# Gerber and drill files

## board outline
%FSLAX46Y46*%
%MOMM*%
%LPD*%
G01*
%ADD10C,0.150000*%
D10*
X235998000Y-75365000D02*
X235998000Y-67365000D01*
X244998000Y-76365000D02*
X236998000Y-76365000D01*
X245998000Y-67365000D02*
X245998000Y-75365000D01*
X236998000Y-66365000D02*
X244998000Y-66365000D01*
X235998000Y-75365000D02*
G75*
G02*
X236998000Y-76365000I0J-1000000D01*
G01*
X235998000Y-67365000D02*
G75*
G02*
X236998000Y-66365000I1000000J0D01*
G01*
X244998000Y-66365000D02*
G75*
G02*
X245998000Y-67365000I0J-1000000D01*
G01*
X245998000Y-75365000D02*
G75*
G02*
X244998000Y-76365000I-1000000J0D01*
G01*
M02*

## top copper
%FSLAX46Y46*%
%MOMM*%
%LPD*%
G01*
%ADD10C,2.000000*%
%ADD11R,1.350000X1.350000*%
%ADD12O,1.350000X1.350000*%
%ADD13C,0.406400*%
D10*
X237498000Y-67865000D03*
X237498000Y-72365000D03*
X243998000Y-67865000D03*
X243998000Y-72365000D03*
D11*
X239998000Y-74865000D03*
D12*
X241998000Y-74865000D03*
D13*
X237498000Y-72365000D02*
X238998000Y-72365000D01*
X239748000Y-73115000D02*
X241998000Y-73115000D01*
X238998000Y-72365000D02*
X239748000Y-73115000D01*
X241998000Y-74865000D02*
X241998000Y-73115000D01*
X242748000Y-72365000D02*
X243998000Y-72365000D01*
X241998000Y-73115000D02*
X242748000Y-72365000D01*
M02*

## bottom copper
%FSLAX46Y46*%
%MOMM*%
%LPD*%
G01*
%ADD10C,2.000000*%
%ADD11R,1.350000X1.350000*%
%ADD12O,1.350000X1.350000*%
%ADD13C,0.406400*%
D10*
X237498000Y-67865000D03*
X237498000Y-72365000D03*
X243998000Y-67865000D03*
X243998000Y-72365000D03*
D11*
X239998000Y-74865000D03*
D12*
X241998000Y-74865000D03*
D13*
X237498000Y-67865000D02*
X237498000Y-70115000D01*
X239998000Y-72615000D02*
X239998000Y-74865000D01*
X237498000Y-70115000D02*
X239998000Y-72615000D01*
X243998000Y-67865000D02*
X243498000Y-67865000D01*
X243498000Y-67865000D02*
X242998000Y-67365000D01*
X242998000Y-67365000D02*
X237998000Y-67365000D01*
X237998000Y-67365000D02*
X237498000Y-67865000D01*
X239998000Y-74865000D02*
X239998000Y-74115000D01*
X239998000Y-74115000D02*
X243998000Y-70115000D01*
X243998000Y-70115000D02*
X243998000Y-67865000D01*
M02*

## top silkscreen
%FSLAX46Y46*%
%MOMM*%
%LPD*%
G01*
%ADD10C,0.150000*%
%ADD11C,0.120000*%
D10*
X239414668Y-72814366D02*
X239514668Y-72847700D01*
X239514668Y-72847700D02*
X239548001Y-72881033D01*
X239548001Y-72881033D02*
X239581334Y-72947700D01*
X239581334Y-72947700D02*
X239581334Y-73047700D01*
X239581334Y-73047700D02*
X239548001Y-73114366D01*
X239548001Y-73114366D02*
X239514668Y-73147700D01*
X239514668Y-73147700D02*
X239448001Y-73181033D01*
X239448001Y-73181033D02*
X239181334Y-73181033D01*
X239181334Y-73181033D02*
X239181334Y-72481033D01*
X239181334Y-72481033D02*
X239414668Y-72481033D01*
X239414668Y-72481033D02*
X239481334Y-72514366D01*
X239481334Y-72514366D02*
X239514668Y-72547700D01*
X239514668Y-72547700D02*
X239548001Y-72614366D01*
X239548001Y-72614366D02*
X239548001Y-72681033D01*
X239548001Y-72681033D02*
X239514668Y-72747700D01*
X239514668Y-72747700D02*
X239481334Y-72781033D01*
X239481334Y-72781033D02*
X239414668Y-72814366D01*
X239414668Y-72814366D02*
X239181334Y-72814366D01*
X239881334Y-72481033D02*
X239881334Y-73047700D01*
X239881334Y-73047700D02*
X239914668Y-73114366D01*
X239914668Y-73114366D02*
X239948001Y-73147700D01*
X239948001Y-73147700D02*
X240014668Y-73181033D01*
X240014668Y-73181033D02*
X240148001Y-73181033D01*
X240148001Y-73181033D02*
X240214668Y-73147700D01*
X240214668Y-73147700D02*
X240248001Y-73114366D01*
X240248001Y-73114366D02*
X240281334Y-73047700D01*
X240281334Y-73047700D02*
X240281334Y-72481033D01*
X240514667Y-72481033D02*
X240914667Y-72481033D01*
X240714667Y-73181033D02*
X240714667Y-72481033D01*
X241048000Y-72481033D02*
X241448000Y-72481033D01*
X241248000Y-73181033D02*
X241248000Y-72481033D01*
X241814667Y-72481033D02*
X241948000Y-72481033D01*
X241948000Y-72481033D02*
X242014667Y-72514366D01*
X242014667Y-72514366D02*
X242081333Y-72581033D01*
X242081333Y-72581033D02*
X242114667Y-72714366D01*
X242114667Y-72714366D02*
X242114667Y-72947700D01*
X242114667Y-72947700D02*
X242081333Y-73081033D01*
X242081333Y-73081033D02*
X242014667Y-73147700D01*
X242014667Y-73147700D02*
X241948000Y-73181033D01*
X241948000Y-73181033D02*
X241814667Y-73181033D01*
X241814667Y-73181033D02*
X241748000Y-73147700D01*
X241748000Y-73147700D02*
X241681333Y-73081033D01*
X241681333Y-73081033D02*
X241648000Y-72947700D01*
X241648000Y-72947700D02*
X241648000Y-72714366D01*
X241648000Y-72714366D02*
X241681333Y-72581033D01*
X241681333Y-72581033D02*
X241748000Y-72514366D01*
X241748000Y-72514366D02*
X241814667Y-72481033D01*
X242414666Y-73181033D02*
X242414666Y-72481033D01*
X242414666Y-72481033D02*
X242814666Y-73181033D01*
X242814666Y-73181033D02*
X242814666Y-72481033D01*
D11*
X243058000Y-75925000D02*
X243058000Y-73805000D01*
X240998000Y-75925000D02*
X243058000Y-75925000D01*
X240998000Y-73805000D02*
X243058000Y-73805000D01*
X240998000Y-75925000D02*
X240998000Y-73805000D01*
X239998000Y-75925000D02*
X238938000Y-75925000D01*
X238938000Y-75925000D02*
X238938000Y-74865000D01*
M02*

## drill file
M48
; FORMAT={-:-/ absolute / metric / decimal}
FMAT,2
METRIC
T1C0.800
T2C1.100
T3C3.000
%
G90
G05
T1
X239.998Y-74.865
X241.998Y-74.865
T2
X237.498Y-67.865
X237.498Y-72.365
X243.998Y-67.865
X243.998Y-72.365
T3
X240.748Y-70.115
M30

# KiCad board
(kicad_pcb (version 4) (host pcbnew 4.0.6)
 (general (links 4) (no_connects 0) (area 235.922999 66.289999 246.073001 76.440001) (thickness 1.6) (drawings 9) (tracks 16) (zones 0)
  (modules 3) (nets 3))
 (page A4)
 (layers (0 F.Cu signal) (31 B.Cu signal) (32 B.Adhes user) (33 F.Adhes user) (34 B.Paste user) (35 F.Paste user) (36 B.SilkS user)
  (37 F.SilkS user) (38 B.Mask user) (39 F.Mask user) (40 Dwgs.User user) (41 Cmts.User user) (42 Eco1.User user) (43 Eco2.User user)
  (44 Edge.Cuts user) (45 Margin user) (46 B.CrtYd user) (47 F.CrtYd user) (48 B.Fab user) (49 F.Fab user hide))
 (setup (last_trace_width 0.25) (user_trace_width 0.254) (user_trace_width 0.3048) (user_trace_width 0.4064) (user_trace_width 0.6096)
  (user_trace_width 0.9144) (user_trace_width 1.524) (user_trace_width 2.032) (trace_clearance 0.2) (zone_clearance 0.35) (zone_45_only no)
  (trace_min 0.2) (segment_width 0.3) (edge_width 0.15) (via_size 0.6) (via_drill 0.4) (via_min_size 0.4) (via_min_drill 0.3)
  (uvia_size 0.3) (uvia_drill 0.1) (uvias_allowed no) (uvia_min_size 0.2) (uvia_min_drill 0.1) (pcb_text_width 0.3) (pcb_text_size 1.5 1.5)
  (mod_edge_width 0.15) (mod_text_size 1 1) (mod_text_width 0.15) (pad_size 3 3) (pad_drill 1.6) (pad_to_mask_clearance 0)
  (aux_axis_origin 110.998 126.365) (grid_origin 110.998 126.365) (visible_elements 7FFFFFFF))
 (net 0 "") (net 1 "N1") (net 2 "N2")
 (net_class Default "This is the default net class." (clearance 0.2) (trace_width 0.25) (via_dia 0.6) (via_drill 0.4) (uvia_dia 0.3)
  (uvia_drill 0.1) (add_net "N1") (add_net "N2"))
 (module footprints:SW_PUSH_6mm (layer B.Cu) (at 237.498 72.365)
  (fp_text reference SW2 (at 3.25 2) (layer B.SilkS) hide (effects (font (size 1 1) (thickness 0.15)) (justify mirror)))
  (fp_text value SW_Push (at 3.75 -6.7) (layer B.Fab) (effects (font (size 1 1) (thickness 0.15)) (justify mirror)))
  (pad 2 thru_hole circle (at 0 -4.5 270) (size 2 2) (drill 1.1) (layers *.Cu *.Mask) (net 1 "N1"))
  (pad 1 thru_hole circle (at 0 0 270) (size 2 2) (drill 1.1) (layers *.Cu *.Mask) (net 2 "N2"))
  (pad 2 thru_hole circle (at 6.5 -4.5 270) (size 2 2) (drill 1.1) (layers *.Cu *.Mask) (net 1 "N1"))
  (pad 1 thru_hole circle (at 6.5 0 270) (size 2 2) (drill 1.1) (layers *.Cu *.Mask) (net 2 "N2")))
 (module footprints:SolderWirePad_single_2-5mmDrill (layer F.Cu) (at 240.748 70.115)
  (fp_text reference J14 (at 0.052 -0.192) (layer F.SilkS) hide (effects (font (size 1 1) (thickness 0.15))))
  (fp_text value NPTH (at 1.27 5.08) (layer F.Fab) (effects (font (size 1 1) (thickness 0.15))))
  (pad "" np_thru_hole circle (at 0 0) (size 3 3) (drill 3) (layers *.Cu *.Mask)))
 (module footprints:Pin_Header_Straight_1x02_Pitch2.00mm (layer F.Cu) (at 239.998 74.865 90)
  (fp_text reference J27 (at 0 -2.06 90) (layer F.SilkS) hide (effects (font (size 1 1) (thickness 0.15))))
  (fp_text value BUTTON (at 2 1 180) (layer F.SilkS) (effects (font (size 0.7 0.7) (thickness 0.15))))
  (fp_line (start -1.06 3.06) (end 1.06 3.06) (layer F.SilkS) (width 0.12))
  (fp_line (start -1.06 1) (end -1.06 3.06) (layer F.SilkS) (width 0.12))
  (fp_line (start 1.06 1) (end 1.06 3.06) (layer F.SilkS) (width 0.12))
  (fp_line (start -1.06 1) (end 1.06 1) (layer F.SilkS) (width 0.12))
  (fp_line (start -1.06 0) (end -1.06 -1.06) (layer F.SilkS) (width 0.12))
  (fp_line (start -1.06 -1.06) (end 0 -1.06) (layer F.SilkS) (width 0.12))
  (pad 1 thru_hole rect (at 0 0 90) (size 1.35 1.35) (drill 0.8) (layers *.Cu *.Mask) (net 1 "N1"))
  (pad 2 thru_hole oval (at 0 2 90) (size 1.35 1.35) (drill 0.8) (layers *.Cu *.Mask) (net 2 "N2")))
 (gr_line (start 235.998 75.365) (end 235.998 67.365) (angle 90) (layer Edge.Cuts) (width 0.15))
 (gr_line (start 244.998 76.365) (end 236.998 76.365) (angle 90) (layer Edge.Cuts) (width 0.15))
 (gr_line (start 245.998 67.365) (end 245.998 75.365) (angle 90) (layer Edge.Cuts) (width 0.15))
 (gr_line (start 236.998 66.365) (end 244.998 66.365) (angle 90) (layer Edge.Cuts) (width 0.15))
 (gr_arc (start 235.998 76.365) (end 235.998 75.365) (angle 90) (layer Edge.Cuts) (width 0.15))
 (gr_arc (start 236.998 67.365) (end 235.998 67.365) (angle 90) (layer Edge.Cuts) (width 0.15))
 (gr_arc (start 244.998 67.365) (end 244.998 66.365) (angle 90) (layer Edge.Cuts) (width 0.15))
 (gr_arc (start 244.998 75.365) (end 245.998 75.365) (angle 90) (layer Edge.Cuts) (width 0.15))
 (segment (start 237.498 67.865) (end 237.498 70.115) (width 0.4064) (layer B.Cu) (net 1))
 (segment (start 239.998 72.615) (end 239.998 74.865) (width 0.4064) (layer B.Cu) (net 1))
 (segment (start 237.498 70.115) (end 239.998 72.615) (width 0.4064) (layer B.Cu) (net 1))
 (segment (start 243.998 67.865) (end 243.498 67.865) (width 0.4064) (layer B.Cu) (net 1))
 (segment (start 243.498 67.865) (end 242.998 67.365) (width 0.4064) (layer B.Cu) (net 1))
 (segment (start 242.998 67.365) (end 237.998 67.365) (width 0.4064) (layer B.Cu) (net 1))
 (segment (start 237.998 67.365) (end 237.498 67.865) (width 0.4064) (layer B.Cu) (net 1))
 (segment (start 239.998 74.865) (end 239.998 74.115) (width 0.4064) (layer B.Cu) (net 1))
 (segment (start 239.998 74.115) (end 243.998 70.115) (width 0.4064) (layer B.Cu) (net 1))
 (segment (start 243.998 70.115) (end 243.998 67.865) (width 0.4064) (layer B.Cu) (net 1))
 (segment (start 237.498 72.365) (end 238.998 72.365) (width 0.4064) (layer F.Cu) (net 2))
 (segment (start 239.748 73.115) (end 241.998 73.115) (width 0.4064) (layer F.Cu) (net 2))
 (segment (start 238.998 72.365) (end 239.748 73.115) (width 0.4064) (layer F.Cu) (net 2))
 (segment (start 241.998 74.865) (end 241.998 73.115) (width 0.4064) (layer F.Cu) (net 2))
 (segment (start 242.748 72.365) (end 243.998 72.365) (width 0.4064) (layer F.Cu) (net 2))
 (segment (start 241.998 73.115) (end 242.748 72.365) (width 0.4064) (layer F.Cu) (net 2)))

